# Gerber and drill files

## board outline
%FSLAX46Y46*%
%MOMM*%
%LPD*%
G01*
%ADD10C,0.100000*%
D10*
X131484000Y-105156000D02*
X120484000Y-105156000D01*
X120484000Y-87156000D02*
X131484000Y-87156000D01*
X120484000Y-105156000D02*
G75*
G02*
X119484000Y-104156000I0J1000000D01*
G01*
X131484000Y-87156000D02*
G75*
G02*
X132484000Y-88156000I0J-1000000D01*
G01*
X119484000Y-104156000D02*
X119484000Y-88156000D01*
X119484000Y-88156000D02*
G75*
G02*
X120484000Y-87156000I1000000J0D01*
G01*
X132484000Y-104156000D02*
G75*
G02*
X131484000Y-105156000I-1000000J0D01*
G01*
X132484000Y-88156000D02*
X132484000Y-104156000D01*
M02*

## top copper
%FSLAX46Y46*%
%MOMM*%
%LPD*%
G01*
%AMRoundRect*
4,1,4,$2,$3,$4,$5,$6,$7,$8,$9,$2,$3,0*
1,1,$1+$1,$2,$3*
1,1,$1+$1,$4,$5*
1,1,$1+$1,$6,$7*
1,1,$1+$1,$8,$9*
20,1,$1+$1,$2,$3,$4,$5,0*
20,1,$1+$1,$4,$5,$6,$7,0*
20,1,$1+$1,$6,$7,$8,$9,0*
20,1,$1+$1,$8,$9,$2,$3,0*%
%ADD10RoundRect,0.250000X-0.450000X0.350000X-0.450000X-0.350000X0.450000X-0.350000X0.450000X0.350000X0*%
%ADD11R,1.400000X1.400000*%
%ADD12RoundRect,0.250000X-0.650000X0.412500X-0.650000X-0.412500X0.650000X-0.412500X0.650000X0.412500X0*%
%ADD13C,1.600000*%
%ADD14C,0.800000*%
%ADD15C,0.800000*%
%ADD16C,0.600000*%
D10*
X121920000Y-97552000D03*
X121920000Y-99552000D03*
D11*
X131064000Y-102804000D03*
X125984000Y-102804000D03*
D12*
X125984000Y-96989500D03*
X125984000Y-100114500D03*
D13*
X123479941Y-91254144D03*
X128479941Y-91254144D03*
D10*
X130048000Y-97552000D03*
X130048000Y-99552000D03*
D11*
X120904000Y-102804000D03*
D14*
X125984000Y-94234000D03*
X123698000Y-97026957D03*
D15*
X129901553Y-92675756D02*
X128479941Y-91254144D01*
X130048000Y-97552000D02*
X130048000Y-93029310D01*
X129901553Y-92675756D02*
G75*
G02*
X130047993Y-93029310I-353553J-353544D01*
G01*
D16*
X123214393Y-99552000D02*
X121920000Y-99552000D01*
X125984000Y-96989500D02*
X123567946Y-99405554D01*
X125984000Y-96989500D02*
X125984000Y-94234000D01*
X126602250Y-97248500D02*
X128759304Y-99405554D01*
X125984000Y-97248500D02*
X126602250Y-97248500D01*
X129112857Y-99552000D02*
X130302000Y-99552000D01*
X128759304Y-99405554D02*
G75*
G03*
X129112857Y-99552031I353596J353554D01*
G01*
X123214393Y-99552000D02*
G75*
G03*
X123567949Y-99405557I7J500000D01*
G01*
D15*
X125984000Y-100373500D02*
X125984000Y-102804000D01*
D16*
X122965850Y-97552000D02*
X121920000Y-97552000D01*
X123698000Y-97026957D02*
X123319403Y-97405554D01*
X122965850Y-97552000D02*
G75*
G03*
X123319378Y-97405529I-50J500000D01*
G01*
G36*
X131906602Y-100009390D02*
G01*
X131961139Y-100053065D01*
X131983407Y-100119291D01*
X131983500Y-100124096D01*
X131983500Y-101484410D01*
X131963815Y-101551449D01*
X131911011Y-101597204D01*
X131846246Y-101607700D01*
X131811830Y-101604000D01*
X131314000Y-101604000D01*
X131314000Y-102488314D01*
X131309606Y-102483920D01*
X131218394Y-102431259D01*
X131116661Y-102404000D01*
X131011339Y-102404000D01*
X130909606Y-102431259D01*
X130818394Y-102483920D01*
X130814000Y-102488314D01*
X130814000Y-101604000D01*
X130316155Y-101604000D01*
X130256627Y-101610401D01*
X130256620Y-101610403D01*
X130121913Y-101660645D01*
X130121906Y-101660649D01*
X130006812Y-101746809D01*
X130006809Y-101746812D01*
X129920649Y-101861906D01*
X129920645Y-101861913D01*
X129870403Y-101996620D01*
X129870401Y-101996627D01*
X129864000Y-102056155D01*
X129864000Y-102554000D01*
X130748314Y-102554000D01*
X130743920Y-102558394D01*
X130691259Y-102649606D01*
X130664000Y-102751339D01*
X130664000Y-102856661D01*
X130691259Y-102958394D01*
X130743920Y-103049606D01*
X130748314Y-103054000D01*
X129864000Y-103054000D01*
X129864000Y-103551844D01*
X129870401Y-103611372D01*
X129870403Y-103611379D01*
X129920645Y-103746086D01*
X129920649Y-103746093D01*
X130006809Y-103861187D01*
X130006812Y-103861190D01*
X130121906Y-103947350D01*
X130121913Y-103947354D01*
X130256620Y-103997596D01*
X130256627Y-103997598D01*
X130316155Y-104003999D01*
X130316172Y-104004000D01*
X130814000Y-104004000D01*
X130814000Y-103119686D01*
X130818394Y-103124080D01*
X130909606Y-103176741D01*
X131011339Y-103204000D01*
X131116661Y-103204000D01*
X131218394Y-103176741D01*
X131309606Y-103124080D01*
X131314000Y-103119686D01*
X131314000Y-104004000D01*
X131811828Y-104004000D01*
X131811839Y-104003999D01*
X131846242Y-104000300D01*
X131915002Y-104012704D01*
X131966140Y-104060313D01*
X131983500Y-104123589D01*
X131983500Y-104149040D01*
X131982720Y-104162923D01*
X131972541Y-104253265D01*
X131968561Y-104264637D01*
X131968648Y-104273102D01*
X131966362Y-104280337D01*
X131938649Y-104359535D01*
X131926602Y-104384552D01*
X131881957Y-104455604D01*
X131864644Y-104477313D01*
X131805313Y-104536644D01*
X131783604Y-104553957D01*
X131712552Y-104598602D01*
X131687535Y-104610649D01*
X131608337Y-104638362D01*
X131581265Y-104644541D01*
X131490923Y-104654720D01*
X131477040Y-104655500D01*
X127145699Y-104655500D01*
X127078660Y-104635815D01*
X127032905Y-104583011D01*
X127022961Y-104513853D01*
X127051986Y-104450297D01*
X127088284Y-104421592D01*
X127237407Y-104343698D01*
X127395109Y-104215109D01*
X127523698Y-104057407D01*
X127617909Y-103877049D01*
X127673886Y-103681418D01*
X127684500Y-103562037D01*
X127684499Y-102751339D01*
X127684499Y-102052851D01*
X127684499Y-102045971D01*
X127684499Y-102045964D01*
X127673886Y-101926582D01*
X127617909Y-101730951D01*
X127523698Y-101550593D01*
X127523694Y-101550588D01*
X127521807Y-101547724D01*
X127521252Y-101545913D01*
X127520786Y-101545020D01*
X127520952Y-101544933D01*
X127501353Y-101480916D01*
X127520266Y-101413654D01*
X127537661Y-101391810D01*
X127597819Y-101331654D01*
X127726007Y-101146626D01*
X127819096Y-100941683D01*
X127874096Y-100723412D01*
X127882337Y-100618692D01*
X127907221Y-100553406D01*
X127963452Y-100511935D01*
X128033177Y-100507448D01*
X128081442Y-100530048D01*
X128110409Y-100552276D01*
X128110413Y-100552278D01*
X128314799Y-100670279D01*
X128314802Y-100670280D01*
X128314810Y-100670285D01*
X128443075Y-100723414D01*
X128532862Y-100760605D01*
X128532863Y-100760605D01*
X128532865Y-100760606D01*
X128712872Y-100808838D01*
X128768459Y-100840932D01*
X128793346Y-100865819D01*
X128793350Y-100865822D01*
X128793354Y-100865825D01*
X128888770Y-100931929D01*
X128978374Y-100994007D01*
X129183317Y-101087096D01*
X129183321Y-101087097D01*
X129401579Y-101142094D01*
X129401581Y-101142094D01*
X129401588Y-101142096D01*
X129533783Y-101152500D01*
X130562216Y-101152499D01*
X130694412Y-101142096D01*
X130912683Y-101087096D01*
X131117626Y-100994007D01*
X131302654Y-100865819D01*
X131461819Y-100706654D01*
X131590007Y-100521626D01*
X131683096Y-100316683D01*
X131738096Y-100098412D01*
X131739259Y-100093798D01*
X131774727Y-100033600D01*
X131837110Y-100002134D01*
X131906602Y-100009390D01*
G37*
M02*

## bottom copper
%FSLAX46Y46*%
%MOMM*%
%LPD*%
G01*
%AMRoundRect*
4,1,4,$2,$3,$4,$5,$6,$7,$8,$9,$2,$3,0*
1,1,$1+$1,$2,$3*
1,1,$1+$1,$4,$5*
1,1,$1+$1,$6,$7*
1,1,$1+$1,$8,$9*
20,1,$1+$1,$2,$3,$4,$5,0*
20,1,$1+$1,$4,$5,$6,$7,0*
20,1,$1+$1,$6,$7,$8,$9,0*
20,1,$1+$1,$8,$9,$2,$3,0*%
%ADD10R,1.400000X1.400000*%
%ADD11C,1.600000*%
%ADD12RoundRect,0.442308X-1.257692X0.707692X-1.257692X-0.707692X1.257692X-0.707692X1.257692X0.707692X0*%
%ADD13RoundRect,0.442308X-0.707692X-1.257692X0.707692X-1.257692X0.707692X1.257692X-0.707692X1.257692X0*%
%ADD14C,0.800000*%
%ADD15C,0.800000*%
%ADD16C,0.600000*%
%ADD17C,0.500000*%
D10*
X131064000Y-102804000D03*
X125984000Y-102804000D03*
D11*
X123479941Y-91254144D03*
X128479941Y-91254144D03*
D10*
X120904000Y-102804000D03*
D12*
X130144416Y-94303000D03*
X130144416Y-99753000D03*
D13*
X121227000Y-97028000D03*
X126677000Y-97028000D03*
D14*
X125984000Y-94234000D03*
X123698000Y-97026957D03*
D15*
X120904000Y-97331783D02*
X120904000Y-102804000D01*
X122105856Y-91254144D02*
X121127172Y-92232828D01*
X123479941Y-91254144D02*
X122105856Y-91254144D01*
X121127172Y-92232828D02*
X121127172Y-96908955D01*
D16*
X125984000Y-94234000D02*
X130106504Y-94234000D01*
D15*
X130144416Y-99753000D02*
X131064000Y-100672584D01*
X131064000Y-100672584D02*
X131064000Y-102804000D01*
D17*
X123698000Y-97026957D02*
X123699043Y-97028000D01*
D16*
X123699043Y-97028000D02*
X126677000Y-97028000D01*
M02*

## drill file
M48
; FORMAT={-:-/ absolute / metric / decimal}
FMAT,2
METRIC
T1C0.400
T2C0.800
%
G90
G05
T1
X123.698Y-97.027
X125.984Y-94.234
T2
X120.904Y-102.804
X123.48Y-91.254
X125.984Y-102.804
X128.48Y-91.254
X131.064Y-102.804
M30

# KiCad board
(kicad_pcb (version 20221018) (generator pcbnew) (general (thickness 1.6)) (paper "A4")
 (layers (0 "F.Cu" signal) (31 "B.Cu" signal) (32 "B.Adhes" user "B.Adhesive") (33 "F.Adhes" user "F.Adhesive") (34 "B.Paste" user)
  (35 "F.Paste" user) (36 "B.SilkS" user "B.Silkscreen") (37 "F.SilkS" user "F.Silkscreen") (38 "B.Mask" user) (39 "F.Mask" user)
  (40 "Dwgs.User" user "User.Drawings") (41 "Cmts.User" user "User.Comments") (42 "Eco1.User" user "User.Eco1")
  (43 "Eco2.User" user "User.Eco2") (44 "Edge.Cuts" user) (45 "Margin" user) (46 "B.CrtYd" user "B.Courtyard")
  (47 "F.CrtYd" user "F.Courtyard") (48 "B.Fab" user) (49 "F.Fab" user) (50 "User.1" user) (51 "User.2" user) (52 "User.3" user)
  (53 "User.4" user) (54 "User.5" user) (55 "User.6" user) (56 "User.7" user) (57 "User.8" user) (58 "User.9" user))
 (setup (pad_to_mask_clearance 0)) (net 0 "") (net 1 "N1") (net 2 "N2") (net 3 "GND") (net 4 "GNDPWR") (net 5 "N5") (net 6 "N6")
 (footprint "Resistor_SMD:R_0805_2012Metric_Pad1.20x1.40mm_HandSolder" (layer "F.Cu") (at 121.92 98.552 -90)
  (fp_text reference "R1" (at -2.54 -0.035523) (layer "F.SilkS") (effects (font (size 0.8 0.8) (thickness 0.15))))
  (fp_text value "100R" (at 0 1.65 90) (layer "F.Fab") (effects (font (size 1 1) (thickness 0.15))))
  (pad "1" smd roundrect (at -1 0 270) (size 1.2 1.4) (layers "F.Cu" "F.Paste" "F.Mask") (roundrect_rratio 0.2083333333) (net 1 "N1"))
  (pad "2" smd roundrect (at 1 0 270) (size 1.2 1.4) (layers "F.Cu" "F.Paste" "F.Mask") (roundrect_rratio 0.2083333333) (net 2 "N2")))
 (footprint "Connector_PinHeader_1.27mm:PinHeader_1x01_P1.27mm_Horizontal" (layer "F.Cu") (at 131.064 102.804 -90)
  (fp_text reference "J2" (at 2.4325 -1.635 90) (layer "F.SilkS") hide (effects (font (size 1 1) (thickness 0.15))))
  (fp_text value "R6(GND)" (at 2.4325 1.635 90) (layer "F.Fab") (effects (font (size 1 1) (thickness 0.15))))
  (pad "1" thru_hole rect (at 0 0 270) (size 1.4 1.4) (drill 0.8) (layers "*.Cu" "*.Mask") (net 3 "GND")))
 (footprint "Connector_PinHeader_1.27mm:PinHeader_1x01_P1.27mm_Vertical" (layer "F.Cu") (at 125.984 102.804)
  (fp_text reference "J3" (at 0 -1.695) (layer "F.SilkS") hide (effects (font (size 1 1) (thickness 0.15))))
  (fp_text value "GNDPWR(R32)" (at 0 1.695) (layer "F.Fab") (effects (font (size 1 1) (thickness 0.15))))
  (pad "1" thru_hole rect (at 0 0) (size 1.4 1.4) (drill 0.8) (layers "*.Cu" "*.Mask") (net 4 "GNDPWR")))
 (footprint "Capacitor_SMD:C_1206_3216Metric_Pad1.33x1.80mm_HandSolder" (layer "F.Cu") (at 125.984 98.552 -90)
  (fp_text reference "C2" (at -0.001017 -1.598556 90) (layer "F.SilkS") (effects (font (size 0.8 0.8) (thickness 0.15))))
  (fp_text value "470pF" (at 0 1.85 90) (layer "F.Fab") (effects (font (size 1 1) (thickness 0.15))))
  (pad "1" smd roundrect (at -1.5625 0 270) (size 1.325 1.8) (layers "F.Cu" "F.Paste" "F.Mask") (roundrect_rratio 0.1886792453) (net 2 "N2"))
  (pad "2" smd roundrect (at 1.5625 0 270) (size 1.325 1.8) (layers "F.Cu" "F.Paste" "F.Mask") (roundrect_rratio 0.1886792453)
   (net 4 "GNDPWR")))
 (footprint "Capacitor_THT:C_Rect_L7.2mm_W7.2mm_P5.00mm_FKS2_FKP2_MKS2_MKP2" (layer "F.Cu") (at 123.479941 91.254144)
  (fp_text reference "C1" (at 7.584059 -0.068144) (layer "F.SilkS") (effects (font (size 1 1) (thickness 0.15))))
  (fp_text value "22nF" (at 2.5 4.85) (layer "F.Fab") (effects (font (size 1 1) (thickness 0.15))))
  (pad "1" thru_hole circle (at 0 0) (size 1.6 1.6) (drill 0.8) (layers "*.Cu" "*.Mask") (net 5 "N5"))
  (pad "2" thru_hole circle (at 5 0) (size 1.6 1.6) (drill 0.8) (layers "*.Cu" "*.Mask") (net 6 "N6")))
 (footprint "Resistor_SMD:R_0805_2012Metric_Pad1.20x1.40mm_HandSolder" (layer "F.Cu") (at 130.048 98.552 -90)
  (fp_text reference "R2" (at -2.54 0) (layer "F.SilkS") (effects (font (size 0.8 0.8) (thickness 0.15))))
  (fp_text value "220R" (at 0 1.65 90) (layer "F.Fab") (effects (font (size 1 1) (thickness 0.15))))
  (pad "1" smd roundrect (at -1 0 270) (size 1.2 1.4) (layers "F.Cu" "F.Paste" "F.Mask") (roundrect_rratio 0.2083333333) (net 6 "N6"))
  (pad "2" smd roundrect (at 1 0 270) (size 1.2 1.4) (layers "F.Cu" "F.Paste" "F.Mask") (roundrect_rratio 0.2083333333) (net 2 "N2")))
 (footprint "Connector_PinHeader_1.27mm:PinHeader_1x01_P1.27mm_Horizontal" (layer "F.Cu") (at 120.904 102.804 -90)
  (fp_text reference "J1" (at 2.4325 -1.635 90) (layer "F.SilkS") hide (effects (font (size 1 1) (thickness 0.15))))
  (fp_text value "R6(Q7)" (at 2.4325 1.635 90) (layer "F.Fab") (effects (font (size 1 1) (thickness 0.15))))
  (pad "1" thru_hole rect (at 0 0 270) (size 1.4 1.4) (drill 0.8) (layers "*.Cu" "*.Mask") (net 5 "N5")))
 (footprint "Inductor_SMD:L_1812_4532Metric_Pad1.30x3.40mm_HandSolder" (layer "B.Cu") (at 130.144416 97.028 -90)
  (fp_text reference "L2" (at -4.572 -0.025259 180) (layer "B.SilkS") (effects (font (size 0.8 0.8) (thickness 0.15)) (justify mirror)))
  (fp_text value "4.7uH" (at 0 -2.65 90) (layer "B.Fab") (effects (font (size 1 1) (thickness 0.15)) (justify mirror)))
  (pad "1" smd roundrect (at -2.725 0 270) (size 2.3 3.4) (layers "B.Cu" "B.Paste" "B.Mask") (roundrect_rratio 0.1923078261) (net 2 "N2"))
  (pad "2" smd roundrect (at 2.725 0 270) (size 2.3 3.4) (layers "B.Cu" "B.Paste" "B.Mask") (roundrect_rratio 0.1923078261) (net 3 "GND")))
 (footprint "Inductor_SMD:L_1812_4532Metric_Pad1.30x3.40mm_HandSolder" (layer "B.Cu") (at 123.952 97.028)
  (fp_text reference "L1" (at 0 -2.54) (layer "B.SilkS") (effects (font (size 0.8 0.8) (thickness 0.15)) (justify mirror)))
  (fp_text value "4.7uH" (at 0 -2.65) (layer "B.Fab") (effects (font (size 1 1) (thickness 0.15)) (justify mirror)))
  (pad "1" smd roundrect (at -2.725 0) (size 2.3 3.4) (layers "B.Cu" "B.Paste" "B.Mask") (roundrect_rratio 0.1923078261) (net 5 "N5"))
  (pad "2" smd roundrect (at 2.725 0) (size 2.3 3.4) (layers "B.Cu" "B.Paste" "B.Mask") (roundrect_rratio 0.1923078261) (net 1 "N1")))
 (gr_line (start 131.484 105.156) (end 120.484 105.156) (stroke (width 0.1) (type default)) (layer "Edge.Cuts"))
 (gr_line (start 120.484 87.156) (end 131.484 87.156) (stroke (width 0.1) (type default)) (layer "Edge.Cuts"))
 (gr_arc (start 120.484 105.156) (mid 119.776893 104.863107) (end 119.484 104.156) (stroke (width 0.1) (type default)) (layer "Edge.Cuts"))
 (gr_arc (start 131.484 87.156) (mid 132.191107 87.448893) (end 132.484 88.156) (stroke (width 0.1) (type default)) (layer "Edge.Cuts"))
 (gr_line (start 119.484 104.156) (end 119.484 88.156) (stroke (width 0.1) (type default)) (layer "Edge.Cuts"))
 (gr_arc (start 119.484 88.156) (mid 119.776893 87.448893) (end 120.484 87.156) (stroke (width 0.1) (type default)) (layer "Edge.Cuts"))
 (gr_arc (start 132.484 104.156) (mid 132.191107 104.863107) (end 131.484 105.156) (stroke (width 0.1) (type default)) (layer "Edge.Cuts"))
 (gr_line (start 132.484 88.156) (end 132.484 104.156) (stroke (width 0.1) (type default)) (layer "Edge.Cuts"))
 (segment (start 120.904 97.331783) (end 120.904 102.804) (width 0.8) (layer "B.Cu") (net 5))
 (segment (start 122.105856 91.254144) (end 121.127172 92.232828) (width 0.8) (layer "B.Cu") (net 5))
 (segment (start 123.479941 91.254144) (end 122.105856 91.254144) (width 0.8) (layer "B.Cu") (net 5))
 (segment (start 121.127172 92.232828) (end 121.127172 96.908955) (width 0.8) (layer "B.Cu") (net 5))
 (segment (start 129.901553 92.675756) (end 128.479941 91.254144) (width 0.8) (layer "F.Cu") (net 6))
 (segment (start 130.048 97.552) (end 130.048 93.02931) (width 0.8) (layer "F.Cu") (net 6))
 (arc (start 129.901553 92.675756) (mid 130.00994 92.837968) (end 130.048 93.02931) (width 0.8) (layer "F.Cu") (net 6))
 (segment (start 123.214393 99.552) (end 121.92 99.552) (width 0.6) (layer "F.Cu") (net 2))
 (segment (start 125.984 96.9895) (end 123.567946 99.405554) (width 0.6) (layer "F.Cu") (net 2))
 (segment (start 125.984 96.9895) (end 125.984 94.234) (width 0.6) (layer "F.Cu") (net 2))
 (segment (start 126.60225 97.2485) (end 128.759304 99.405554) (width 0.6) (layer "F.Cu") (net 2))
 (segment (start 125.984 97.2485) (end 126.60225 97.2485) (width 0.6) (layer "F.Cu") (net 2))
 (segment (start 129.112857 99.552) (end 130.302 99.552) (width 0.6) (layer "F.Cu") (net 2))
 (via (at 125.984 94.234) (size 0.8) (drill 0.4) (layers "F.Cu" "B.Cu") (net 2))
 (arc (start 128.759304 99.405554) (mid 128.921516 99.51394) (end 129.112857 99.552) (width 0.6) (layer "F.Cu") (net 2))
 (arc (start 123.214393 99.552) (mid 123.405734 99.51394) (end 123.567946 99.405554) (width 0.6) (layer "F.Cu") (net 2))
 (segment (start 125.984 94.234) (end 130.106504 94.234) (width 0.6) (layer "B.Cu") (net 2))
 (segment (start 125.984 100.3735) (end 125.984 102.804) (width 0.8) (layer "F.Cu") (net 4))
 (segment (start 130.144416 99.753) (end 131.064 100.672584) (width 0.8) (layer "B.Cu") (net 3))
 (segment (start 131.064 100.672584) (end 131.064 102.804) (width 0.8) (layer "B.Cu") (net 3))
 (segment (start 122.96585 97.552) (end 121.92 97.552) (width 0.6) (layer "F.Cu") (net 1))
 (segment (start 123.698 97.026957) (end 123.319403 97.405554) (width 0.6) (layer "F.Cu") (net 1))
 (via (at 123.698 97.026957) (size 0.8) (drill 0.4) (layers "F.Cu" "B.Cu") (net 1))
 (arc (start 122.96585 97.552) (mid 123.157191 97.51394) (end 123.319403 97.405554) (width 0.6) (layer "F.Cu") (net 1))
 (segment (start 123.698 97.026957) (end 123.699043 97.028) (width 0.5) (layer "B.Cu") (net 1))
 (segment (start 123.699043 97.028) (end 126.677 97.028) (width 0.6) (layer "B.Cu") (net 1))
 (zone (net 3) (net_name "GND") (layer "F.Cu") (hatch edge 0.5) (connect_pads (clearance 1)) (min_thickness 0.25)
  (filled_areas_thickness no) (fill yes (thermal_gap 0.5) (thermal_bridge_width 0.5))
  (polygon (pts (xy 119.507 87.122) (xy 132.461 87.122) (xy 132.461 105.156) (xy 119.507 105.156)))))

